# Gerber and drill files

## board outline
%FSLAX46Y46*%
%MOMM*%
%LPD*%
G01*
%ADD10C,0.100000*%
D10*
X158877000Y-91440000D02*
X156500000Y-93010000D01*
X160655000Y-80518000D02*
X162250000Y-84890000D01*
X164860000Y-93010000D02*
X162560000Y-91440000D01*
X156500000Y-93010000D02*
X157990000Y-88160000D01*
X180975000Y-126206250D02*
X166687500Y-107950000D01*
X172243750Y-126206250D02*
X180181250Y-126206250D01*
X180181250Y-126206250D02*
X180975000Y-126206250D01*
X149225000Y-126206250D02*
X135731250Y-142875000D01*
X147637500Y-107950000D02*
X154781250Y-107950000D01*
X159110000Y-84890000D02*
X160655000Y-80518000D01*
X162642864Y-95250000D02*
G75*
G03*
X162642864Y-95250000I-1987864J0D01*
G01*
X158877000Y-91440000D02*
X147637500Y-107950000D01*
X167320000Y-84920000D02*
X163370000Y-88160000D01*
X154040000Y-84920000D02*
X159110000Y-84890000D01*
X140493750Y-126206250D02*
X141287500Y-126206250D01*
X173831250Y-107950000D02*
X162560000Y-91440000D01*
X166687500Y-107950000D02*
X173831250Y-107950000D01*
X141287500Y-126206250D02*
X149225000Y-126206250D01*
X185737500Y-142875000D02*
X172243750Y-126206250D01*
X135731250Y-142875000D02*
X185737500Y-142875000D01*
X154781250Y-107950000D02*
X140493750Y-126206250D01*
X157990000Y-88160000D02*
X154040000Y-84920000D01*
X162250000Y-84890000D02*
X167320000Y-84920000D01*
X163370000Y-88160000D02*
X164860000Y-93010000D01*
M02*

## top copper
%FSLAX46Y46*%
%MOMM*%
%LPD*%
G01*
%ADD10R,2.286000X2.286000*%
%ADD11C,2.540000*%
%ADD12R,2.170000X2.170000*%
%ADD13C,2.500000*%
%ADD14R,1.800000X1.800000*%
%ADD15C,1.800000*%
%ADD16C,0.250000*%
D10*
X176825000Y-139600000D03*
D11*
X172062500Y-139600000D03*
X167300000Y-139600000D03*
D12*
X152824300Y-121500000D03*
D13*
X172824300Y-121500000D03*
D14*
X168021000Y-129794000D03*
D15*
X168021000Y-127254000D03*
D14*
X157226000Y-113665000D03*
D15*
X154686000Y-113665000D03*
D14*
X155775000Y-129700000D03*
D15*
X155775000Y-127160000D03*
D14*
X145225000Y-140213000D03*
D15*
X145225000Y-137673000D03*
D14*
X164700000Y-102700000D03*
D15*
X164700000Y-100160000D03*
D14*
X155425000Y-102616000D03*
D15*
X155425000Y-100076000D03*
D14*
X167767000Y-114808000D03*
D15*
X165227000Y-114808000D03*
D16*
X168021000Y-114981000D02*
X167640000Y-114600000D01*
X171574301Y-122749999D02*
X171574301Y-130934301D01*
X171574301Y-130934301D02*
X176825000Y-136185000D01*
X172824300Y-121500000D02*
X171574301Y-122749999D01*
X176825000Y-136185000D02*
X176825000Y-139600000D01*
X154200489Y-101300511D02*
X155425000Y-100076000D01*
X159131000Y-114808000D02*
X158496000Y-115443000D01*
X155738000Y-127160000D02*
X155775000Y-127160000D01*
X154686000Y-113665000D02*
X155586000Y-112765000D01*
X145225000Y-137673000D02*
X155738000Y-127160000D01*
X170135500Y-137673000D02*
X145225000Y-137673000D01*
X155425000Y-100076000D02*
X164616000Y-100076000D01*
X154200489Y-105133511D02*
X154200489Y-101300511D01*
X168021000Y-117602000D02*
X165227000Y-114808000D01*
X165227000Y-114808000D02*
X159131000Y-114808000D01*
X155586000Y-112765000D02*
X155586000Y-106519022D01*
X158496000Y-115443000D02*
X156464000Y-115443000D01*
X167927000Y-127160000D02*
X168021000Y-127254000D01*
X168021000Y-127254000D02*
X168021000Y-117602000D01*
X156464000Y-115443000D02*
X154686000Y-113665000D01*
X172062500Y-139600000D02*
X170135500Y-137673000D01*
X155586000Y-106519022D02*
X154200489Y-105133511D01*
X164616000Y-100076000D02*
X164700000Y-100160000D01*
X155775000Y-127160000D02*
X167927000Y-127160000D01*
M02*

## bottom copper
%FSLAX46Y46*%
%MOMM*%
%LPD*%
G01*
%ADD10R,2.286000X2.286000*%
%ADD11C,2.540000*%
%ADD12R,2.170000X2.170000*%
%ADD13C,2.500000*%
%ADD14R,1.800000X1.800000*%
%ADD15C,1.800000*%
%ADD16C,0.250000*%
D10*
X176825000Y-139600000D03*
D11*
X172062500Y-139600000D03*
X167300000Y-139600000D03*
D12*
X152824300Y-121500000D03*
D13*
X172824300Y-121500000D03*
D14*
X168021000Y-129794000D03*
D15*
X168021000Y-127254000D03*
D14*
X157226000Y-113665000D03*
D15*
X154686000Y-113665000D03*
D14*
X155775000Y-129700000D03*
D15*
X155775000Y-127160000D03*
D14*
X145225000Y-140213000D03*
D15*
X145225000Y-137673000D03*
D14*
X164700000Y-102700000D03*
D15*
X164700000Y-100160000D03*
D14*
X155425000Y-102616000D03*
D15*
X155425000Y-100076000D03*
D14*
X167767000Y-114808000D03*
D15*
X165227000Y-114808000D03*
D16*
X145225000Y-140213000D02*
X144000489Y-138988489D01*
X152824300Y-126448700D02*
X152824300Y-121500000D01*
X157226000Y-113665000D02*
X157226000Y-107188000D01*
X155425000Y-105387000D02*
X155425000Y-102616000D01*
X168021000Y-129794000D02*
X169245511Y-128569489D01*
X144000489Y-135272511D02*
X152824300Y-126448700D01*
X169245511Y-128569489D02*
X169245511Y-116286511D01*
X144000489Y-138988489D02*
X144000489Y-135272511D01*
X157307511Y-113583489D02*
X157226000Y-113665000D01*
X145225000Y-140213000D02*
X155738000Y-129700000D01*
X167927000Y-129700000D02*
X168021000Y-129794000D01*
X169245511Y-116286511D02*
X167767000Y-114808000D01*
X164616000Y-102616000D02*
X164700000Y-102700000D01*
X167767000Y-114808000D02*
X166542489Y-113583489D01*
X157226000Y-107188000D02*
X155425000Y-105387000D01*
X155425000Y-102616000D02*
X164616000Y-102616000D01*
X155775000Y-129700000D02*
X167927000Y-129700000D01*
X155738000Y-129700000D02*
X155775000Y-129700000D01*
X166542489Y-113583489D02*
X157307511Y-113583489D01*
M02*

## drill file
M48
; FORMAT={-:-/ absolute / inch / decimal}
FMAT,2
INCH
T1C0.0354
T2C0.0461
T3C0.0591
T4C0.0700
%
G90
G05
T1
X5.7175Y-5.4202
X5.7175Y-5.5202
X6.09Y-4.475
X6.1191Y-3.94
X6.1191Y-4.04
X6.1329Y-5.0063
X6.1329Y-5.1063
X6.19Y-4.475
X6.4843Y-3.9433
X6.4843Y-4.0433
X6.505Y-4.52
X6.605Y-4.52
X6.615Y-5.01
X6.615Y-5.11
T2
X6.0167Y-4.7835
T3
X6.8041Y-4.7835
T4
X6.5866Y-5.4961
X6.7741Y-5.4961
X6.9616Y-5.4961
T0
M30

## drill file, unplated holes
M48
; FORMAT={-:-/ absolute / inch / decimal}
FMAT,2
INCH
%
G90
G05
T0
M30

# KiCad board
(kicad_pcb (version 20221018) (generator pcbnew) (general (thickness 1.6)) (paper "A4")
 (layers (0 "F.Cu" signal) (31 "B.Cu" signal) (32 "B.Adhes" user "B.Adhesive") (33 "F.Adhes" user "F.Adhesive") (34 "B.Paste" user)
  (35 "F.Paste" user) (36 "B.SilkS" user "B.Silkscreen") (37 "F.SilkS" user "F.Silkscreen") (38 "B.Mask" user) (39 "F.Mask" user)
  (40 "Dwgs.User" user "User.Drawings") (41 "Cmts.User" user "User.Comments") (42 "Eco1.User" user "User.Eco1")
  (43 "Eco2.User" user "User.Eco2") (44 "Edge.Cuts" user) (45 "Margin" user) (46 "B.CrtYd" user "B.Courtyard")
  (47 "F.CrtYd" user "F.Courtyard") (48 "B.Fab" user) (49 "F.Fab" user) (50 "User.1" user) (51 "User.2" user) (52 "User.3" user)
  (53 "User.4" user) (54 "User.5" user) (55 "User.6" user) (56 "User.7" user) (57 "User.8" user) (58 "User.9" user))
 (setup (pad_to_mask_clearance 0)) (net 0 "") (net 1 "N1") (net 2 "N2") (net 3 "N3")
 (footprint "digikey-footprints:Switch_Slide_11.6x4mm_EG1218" (layer "F.Cu") (at 176.3 139.6 180)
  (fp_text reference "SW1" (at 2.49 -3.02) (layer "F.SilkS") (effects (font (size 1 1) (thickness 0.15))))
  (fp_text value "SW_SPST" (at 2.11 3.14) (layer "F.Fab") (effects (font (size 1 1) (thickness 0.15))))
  (pad "1" thru_hole rect (at -0.525 0 180) (size 2.286 2.286) (drill 1.778) (layers "*.Cu" "*.Mask") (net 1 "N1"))
  (pad "2" thru_hole circle (at 4.2375 0 180) (size 2.54 2.54) (drill 1.778) (layers "*.Cu" "*.Mask") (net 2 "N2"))
  (pad "3" thru_hole circle (at 9 0 180) (size 2.54 2.54) (drill 1.778) (layers "*.Cu" "*.Mask")))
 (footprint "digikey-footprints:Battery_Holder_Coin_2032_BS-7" (layer "F.Cu") (at 152.8243 121.5)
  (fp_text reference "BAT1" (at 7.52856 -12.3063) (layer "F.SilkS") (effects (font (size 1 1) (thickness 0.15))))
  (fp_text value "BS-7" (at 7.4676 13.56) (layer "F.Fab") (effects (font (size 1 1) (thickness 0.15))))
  (pad "Neg" thru_hole rect (at 0 0) (size 2.17 2.17) (drill 1.17) (layers "*.Cu" "*.Mask") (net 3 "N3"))
  (pad "Pos" thru_hole circle (at 20 0) (size 2.5 2.5) (drill 1.5) (layers "*.Cu" "*.Mask") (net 1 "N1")))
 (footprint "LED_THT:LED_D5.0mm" (layer "B.Cu") (at 168.021 129.794 90)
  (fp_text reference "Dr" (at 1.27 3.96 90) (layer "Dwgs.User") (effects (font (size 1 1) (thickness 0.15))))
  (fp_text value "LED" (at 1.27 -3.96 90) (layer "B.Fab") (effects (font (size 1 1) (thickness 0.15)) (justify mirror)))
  (pad "1" thru_hole rect (at 0 0 90) (size 1.8 1.8) (drill 0.9) (layers "*.Cu" "*.Mask") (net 3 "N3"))
  (pad "2" thru_hole circle (at 2.54 0 90) (size 1.8 1.8) (drill 0.9) (layers "*.Cu" "*.Mask") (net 2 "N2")))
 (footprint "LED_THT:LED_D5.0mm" (layer "B.Cu") (at 157.226 113.665 180)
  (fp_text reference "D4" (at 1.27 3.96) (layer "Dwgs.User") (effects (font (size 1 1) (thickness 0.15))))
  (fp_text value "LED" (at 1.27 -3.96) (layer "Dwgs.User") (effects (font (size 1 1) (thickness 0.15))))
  (pad "1" thru_hole rect (at 0 0 180) (size 1.8 1.8) (drill 0.9) (layers "*.Cu" "*.Mask") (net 3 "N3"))
  (pad "2" thru_hole circle (at 2.54 0 180) (size 1.8 1.8) (drill 0.9) (layers "*.Cu" "*.Mask") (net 2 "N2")))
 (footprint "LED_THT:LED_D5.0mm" (layer "B.Cu") (at 155.775 129.7 90)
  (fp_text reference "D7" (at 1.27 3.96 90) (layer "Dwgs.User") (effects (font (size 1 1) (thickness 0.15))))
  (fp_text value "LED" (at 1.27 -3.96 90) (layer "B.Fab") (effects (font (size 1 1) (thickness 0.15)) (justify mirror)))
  (pad "1" thru_hole rect (at 0 0 90) (size 1.8 1.8) (drill 0.9) (layers "*.Cu" "*.Mask") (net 3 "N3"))
  (pad "2" thru_hole circle (at 2.54 0 90) (size 1.8 1.8) (drill 0.9) (layers "*.Cu" "*.Mask") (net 2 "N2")))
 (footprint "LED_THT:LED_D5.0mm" (layer "B.Cu") (at 145.225 140.213 90)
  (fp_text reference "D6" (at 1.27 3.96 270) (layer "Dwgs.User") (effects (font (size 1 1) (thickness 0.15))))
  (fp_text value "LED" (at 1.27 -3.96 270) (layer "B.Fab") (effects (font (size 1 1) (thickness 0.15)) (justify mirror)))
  (pad "1" thru_hole rect (at 0 0 90) (size 1.8 1.8) (drill 0.9) (layers "*.Cu" "*.Mask") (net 3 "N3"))
  (pad "2" thru_hole circle (at 2.54 0 90) (size 1.8 1.8) (drill 0.9) (layers "*.Cu" "*.Mask") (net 2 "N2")))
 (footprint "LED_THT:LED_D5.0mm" (layer "B.Cu") (at 164.7 102.7 90)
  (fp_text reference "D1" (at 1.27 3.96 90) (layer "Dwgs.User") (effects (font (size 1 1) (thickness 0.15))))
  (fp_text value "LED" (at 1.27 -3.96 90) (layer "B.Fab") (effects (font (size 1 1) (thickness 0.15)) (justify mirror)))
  (pad "1" thru_hole rect (at 0 0 90) (size 1.8 1.8) (drill 0.9) (layers "*.Cu" "*.Mask") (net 3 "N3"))
  (pad "2" thru_hole circle (at 2.54 0 90) (size 1.8 1.8) (drill 0.9) (layers "*.Cu" "*.Mask") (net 2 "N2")))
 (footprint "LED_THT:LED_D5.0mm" (layer "B.Cu") (at 155.425 102.616 90)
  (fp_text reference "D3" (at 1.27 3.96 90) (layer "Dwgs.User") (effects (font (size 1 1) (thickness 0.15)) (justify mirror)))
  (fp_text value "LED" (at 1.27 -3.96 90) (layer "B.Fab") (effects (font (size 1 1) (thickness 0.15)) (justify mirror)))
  (pad "1" thru_hole rect (at 0 0 90) (size 1.8 1.8) (drill 0.9) (layers "*.Cu" "*.Mask") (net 3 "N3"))
  (pad "2" thru_hole circle (at 2.54 0 90) (size 1.8 1.8) (drill 0.9) (layers "*.Cu" "*.Mask") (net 2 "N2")))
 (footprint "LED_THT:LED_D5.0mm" (layer "B.Cu") (at 167.767 114.808 180)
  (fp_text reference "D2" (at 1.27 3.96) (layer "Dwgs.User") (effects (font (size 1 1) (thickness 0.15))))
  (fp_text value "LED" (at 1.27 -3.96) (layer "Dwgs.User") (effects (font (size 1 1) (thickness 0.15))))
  (pad "1" thru_hole rect (at 0 0 180) (size 1.8 1.8) (drill 0.9) (layers "*.Cu" "*.Mask") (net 3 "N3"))
  (pad "2" thru_hole circle (at 2.54 0 180) (size 1.8 1.8) (drill 0.9) (layers "*.Cu" "*.Mask") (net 2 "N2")))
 (gr_line (start 158.877 91.44) (end 156.5 93.01) (stroke (width 0.1) (type solid)) (layer "Edge.Cuts"))
 (gr_line (start 160.655 80.518) (end 162.25 84.89) (stroke (width 0.1) (type solid)) (layer "Edge.Cuts"))
 (gr_line (start 164.86 93.01) (end 162.56 91.44) (stroke (width 0.1) (type solid)) (layer "Edge.Cuts"))
 (gr_line (start 156.5 93.01) (end 157.99 88.16) (stroke (width 0.1) (type solid)) (layer "Edge.Cuts"))
 (gr_line (start 180.975 126.20625) (end 166.6875 107.95) (stroke (width 0.1) (type solid)) (layer "Edge.Cuts"))
 (gr_line (start 172.24375 126.20625) (end 180.18125 126.20625) (stroke (width 0.1) (type solid)) (layer "Edge.Cuts"))
 (gr_line (start 180.18125 126.20625) (end 180.975 126.20625) (stroke (width 0.1) (type solid)) (layer "Edge.Cuts"))
 (gr_line (start 149.225 126.20625) (end 135.73125 142.875) (stroke (width 0.1) (type solid)) (layer "Edge.Cuts"))
 (gr_line (start 147.6375 107.95) (end 154.78125 107.95) (stroke (width 0.1) (type solid)) (layer "Edge.Cuts"))
 (gr_line (start 159.11 84.89) (end 160.655 80.518) (stroke (width 0.1) (type solid)) (layer "Edge.Cuts"))
 (gr_circle (center 160.655 95.25) (end 161.544 93.472) (stroke (width 0.1) (type solid)) (fill none) (layer "Edge.Cuts"))
 (gr_line (start 158.877 91.44) (end 147.6375 107.95) (stroke (width 0.1) (type solid)) (layer "Edge.Cuts"))
 (gr_line (start 167.32 84.92) (end 163.37 88.16) (stroke (width 0.1) (type solid)) (layer "Edge.Cuts"))
 (gr_line (start 154.04 84.92) (end 159.11 84.89) (stroke (width 0.1) (type solid)) (layer "Edge.Cuts"))
 (gr_line (start 140.49375 126.20625) (end 141.2875 126.20625) (stroke (width 0.1) (type solid)) (layer "Edge.Cuts"))
 (gr_line (start 173.83125 107.95) (end 162.56 91.44) (stroke (width 0.1) (type solid)) (layer "Edge.Cuts"))
 (gr_line (start 166.6875 107.95) (end 173.83125 107.95) (stroke (width 0.1) (type solid)) (layer "Edge.Cuts"))
 (gr_line (start 141.2875 126.20625) (end 149.225 126.20625) (stroke (width 0.1) (type solid)) (layer "Edge.Cuts"))
 (gr_line (start 185.7375 142.875) (end 172.24375 126.20625) (stroke (width 0.1) (type solid)) (layer "Edge.Cuts"))
 (gr_line (start 135.73125 142.875) (end 185.7375 142.875) (stroke (width 0.1) (type solid)) (layer "Edge.Cuts"))
 (gr_line (start 154.78125 107.95) (end 140.49375 126.20625) (stroke (width 0.1) (type solid)) (layer "Edge.Cuts"))
 (gr_line (start 157.99 88.16) (end 154.04 84.92) (stroke (width 0.1) (type solid)) (layer "Edge.Cuts"))
 (gr_line (start 162.25 84.89) (end 167.32 84.92) (stroke (width 0.1) (type solid)) (layer "Edge.Cuts"))
 (gr_line (start 163.37 88.16) (end 164.86 93.01) (stroke (width 0.1) (type solid)) (layer "Edge.Cuts"))
 (segment (start 168.021 114.981) (end 167.64 114.6) (width 0.25) (layer "F.Cu") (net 3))
 (segment (start 145.225 140.213) (end 144.000489 138.988489) (width 0.25) (layer "B.Cu") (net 3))
 (segment (start 152.8243 126.4487) (end 152.8243 121.5) (width 0.25) (layer "B.Cu") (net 3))
 (segment (start 157.226 113.665) (end 157.226 107.188) (width 0.25) (layer "B.Cu") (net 3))
 (segment (start 155.425 105.387) (end 155.425 102.616) (width 0.25) (layer "B.Cu") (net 3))
 (segment (start 168.021 129.794) (end 169.245511 128.569489) (width 0.25) (layer "B.Cu") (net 3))
 (segment (start 144.000489 135.272511) (end 152.8243 126.4487) (width 0.25) (layer "B.Cu") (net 3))
 (segment (start 169.245511 128.569489) (end 169.245511 116.286511) (width 0.25) (layer "B.Cu") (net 3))
 (segment (start 144.000489 138.988489) (end 144.000489 135.272511) (width 0.25) (layer "B.Cu") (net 3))
 (segment (start 157.307511 113.583489) (end 157.226 113.665) (width 0.25) (layer "B.Cu") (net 3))
 (segment (start 145.225 140.213) (end 155.738 129.7) (width 0.25) (layer "B.Cu") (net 3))
 (segment (start 167.927 129.7) (end 168.021 129.794) (width 0.25) (layer "B.Cu") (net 3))
 (segment (start 169.245511 116.286511) (end 167.767 114.808) (width 0.25) (layer "B.Cu") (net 3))
 (segment (start 164.616 102.616) (end 164.7 102.7) (width 0.25) (layer "B.Cu") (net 3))
 (segment (start 167.767 114.808) (end 166.542489 113.583489) (width 0.25) (layer "B.Cu") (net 3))
 (segment (start 157.226 107.188) (end 155.425 105.387) (width 0.25) (layer "B.Cu") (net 3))
 (segment (start 155.425 102.616) (end 164.616 102.616) (width 0.25) (layer "B.Cu") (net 3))
 (segment (start 155.775 129.7) (end 167.927 129.7) (width 0.25) (layer "B.Cu") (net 3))
 (segment (start 155.738 129.7) (end 155.775 129.7) (width 0.25) (layer "B.Cu") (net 3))
 (segment (start 166.542489 113.583489) (end 157.307511 113.583489) (width 0.25) (layer "B.Cu") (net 3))
 (segment (start 171.574301 122.749999) (end 171.574301 130.934301) (width 0.25) (layer "F.Cu") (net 1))
 (segment (start 171.574301 130.934301) (end 176.825 136.185) (width 0.25) (layer "F.Cu") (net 1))
 (segment (start 172.8243 121.5) (end 171.574301 122.749999) (width 0.25) (layer "F.Cu") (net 1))
 (segment (start 176.825 136.185) (end 176.825 139.6) (width 0.25) (layer "F.Cu") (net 1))
 (segment (start 154.200489 101.300511) (end 155.425 100.076) (width 0.25) (layer "F.Cu") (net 2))
 (segment (start 159.131 114.808) (end 158.496 115.443) (width 0.25) (layer "F.Cu") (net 2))
 (segment (start 155.738 127.16) (end 155.775 127.16) (width 0.25) (layer "F.Cu") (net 2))
 (segment (start 154.686 113.665) (end 155.586 112.765) (width 0.25) (layer "F.Cu") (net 2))
 (segment (start 145.225 137.673) (end 155.738 127.16) (width 0.25) (layer "F.Cu") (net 2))
 (segment (start 170.1355 137.673) (end 145.225 137.673) (width 0.25) (layer "F.Cu") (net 2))
 (segment (start 155.425 100.076) (end 164.616 100.076) (width 0.25) (layer "F.Cu") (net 2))
 (segment (start 154.200489 105.133511) (end 154.200489 101.300511) (width 0.25) (layer "F.Cu") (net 2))
 (segment (start 168.021 117.602) (end 165.227 114.808) (width 0.25) (layer "F.Cu") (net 2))
 (segment (start 165.227 114.808) (end 159.131 114.808) (width 0.25) (layer "F.Cu") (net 2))
 (segment (start 155.586 112.765) (end 155.586 106.519022) (width 0.25) (layer "F.Cu") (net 2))
 (segment (start 158.496 115.443) (end 156.464 115.443) (width 0.25) (layer "F.Cu") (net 2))
 (segment (start 167.927 127.16) (end 168.021 127.254) (width 0.25) (layer "F.Cu") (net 2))
 (segment (start 168.021 127.254) (end 168.021 117.602) (width 0.25) (layer "F.Cu") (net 2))
 (segment (start 156.464 115.443) (end 154.686 113.665) (width 0.25) (layer "F.Cu") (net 2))
 (segment (start 172.0625 139.6) (end 170.1355 137.673) (width 0.25) (layer "F.Cu") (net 2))
 (segment (start 155.586 106.519022) (end 154.200489 105.133511) (width 0.25) (layer "F.Cu") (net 2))
 (segment (start 164.616 100.076) (end 164.7 100.16) (width 0.25) (layer "F.Cu") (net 2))
 (segment (start 155.775 127.16) (end 167.927 127.16) (width 0.25) (layer "F.Cu") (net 2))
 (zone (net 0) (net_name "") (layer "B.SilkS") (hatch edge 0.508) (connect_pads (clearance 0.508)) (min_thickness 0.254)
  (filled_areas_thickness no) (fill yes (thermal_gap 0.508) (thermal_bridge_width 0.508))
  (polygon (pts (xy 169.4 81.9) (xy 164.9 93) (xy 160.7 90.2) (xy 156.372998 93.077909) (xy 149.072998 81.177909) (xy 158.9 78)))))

